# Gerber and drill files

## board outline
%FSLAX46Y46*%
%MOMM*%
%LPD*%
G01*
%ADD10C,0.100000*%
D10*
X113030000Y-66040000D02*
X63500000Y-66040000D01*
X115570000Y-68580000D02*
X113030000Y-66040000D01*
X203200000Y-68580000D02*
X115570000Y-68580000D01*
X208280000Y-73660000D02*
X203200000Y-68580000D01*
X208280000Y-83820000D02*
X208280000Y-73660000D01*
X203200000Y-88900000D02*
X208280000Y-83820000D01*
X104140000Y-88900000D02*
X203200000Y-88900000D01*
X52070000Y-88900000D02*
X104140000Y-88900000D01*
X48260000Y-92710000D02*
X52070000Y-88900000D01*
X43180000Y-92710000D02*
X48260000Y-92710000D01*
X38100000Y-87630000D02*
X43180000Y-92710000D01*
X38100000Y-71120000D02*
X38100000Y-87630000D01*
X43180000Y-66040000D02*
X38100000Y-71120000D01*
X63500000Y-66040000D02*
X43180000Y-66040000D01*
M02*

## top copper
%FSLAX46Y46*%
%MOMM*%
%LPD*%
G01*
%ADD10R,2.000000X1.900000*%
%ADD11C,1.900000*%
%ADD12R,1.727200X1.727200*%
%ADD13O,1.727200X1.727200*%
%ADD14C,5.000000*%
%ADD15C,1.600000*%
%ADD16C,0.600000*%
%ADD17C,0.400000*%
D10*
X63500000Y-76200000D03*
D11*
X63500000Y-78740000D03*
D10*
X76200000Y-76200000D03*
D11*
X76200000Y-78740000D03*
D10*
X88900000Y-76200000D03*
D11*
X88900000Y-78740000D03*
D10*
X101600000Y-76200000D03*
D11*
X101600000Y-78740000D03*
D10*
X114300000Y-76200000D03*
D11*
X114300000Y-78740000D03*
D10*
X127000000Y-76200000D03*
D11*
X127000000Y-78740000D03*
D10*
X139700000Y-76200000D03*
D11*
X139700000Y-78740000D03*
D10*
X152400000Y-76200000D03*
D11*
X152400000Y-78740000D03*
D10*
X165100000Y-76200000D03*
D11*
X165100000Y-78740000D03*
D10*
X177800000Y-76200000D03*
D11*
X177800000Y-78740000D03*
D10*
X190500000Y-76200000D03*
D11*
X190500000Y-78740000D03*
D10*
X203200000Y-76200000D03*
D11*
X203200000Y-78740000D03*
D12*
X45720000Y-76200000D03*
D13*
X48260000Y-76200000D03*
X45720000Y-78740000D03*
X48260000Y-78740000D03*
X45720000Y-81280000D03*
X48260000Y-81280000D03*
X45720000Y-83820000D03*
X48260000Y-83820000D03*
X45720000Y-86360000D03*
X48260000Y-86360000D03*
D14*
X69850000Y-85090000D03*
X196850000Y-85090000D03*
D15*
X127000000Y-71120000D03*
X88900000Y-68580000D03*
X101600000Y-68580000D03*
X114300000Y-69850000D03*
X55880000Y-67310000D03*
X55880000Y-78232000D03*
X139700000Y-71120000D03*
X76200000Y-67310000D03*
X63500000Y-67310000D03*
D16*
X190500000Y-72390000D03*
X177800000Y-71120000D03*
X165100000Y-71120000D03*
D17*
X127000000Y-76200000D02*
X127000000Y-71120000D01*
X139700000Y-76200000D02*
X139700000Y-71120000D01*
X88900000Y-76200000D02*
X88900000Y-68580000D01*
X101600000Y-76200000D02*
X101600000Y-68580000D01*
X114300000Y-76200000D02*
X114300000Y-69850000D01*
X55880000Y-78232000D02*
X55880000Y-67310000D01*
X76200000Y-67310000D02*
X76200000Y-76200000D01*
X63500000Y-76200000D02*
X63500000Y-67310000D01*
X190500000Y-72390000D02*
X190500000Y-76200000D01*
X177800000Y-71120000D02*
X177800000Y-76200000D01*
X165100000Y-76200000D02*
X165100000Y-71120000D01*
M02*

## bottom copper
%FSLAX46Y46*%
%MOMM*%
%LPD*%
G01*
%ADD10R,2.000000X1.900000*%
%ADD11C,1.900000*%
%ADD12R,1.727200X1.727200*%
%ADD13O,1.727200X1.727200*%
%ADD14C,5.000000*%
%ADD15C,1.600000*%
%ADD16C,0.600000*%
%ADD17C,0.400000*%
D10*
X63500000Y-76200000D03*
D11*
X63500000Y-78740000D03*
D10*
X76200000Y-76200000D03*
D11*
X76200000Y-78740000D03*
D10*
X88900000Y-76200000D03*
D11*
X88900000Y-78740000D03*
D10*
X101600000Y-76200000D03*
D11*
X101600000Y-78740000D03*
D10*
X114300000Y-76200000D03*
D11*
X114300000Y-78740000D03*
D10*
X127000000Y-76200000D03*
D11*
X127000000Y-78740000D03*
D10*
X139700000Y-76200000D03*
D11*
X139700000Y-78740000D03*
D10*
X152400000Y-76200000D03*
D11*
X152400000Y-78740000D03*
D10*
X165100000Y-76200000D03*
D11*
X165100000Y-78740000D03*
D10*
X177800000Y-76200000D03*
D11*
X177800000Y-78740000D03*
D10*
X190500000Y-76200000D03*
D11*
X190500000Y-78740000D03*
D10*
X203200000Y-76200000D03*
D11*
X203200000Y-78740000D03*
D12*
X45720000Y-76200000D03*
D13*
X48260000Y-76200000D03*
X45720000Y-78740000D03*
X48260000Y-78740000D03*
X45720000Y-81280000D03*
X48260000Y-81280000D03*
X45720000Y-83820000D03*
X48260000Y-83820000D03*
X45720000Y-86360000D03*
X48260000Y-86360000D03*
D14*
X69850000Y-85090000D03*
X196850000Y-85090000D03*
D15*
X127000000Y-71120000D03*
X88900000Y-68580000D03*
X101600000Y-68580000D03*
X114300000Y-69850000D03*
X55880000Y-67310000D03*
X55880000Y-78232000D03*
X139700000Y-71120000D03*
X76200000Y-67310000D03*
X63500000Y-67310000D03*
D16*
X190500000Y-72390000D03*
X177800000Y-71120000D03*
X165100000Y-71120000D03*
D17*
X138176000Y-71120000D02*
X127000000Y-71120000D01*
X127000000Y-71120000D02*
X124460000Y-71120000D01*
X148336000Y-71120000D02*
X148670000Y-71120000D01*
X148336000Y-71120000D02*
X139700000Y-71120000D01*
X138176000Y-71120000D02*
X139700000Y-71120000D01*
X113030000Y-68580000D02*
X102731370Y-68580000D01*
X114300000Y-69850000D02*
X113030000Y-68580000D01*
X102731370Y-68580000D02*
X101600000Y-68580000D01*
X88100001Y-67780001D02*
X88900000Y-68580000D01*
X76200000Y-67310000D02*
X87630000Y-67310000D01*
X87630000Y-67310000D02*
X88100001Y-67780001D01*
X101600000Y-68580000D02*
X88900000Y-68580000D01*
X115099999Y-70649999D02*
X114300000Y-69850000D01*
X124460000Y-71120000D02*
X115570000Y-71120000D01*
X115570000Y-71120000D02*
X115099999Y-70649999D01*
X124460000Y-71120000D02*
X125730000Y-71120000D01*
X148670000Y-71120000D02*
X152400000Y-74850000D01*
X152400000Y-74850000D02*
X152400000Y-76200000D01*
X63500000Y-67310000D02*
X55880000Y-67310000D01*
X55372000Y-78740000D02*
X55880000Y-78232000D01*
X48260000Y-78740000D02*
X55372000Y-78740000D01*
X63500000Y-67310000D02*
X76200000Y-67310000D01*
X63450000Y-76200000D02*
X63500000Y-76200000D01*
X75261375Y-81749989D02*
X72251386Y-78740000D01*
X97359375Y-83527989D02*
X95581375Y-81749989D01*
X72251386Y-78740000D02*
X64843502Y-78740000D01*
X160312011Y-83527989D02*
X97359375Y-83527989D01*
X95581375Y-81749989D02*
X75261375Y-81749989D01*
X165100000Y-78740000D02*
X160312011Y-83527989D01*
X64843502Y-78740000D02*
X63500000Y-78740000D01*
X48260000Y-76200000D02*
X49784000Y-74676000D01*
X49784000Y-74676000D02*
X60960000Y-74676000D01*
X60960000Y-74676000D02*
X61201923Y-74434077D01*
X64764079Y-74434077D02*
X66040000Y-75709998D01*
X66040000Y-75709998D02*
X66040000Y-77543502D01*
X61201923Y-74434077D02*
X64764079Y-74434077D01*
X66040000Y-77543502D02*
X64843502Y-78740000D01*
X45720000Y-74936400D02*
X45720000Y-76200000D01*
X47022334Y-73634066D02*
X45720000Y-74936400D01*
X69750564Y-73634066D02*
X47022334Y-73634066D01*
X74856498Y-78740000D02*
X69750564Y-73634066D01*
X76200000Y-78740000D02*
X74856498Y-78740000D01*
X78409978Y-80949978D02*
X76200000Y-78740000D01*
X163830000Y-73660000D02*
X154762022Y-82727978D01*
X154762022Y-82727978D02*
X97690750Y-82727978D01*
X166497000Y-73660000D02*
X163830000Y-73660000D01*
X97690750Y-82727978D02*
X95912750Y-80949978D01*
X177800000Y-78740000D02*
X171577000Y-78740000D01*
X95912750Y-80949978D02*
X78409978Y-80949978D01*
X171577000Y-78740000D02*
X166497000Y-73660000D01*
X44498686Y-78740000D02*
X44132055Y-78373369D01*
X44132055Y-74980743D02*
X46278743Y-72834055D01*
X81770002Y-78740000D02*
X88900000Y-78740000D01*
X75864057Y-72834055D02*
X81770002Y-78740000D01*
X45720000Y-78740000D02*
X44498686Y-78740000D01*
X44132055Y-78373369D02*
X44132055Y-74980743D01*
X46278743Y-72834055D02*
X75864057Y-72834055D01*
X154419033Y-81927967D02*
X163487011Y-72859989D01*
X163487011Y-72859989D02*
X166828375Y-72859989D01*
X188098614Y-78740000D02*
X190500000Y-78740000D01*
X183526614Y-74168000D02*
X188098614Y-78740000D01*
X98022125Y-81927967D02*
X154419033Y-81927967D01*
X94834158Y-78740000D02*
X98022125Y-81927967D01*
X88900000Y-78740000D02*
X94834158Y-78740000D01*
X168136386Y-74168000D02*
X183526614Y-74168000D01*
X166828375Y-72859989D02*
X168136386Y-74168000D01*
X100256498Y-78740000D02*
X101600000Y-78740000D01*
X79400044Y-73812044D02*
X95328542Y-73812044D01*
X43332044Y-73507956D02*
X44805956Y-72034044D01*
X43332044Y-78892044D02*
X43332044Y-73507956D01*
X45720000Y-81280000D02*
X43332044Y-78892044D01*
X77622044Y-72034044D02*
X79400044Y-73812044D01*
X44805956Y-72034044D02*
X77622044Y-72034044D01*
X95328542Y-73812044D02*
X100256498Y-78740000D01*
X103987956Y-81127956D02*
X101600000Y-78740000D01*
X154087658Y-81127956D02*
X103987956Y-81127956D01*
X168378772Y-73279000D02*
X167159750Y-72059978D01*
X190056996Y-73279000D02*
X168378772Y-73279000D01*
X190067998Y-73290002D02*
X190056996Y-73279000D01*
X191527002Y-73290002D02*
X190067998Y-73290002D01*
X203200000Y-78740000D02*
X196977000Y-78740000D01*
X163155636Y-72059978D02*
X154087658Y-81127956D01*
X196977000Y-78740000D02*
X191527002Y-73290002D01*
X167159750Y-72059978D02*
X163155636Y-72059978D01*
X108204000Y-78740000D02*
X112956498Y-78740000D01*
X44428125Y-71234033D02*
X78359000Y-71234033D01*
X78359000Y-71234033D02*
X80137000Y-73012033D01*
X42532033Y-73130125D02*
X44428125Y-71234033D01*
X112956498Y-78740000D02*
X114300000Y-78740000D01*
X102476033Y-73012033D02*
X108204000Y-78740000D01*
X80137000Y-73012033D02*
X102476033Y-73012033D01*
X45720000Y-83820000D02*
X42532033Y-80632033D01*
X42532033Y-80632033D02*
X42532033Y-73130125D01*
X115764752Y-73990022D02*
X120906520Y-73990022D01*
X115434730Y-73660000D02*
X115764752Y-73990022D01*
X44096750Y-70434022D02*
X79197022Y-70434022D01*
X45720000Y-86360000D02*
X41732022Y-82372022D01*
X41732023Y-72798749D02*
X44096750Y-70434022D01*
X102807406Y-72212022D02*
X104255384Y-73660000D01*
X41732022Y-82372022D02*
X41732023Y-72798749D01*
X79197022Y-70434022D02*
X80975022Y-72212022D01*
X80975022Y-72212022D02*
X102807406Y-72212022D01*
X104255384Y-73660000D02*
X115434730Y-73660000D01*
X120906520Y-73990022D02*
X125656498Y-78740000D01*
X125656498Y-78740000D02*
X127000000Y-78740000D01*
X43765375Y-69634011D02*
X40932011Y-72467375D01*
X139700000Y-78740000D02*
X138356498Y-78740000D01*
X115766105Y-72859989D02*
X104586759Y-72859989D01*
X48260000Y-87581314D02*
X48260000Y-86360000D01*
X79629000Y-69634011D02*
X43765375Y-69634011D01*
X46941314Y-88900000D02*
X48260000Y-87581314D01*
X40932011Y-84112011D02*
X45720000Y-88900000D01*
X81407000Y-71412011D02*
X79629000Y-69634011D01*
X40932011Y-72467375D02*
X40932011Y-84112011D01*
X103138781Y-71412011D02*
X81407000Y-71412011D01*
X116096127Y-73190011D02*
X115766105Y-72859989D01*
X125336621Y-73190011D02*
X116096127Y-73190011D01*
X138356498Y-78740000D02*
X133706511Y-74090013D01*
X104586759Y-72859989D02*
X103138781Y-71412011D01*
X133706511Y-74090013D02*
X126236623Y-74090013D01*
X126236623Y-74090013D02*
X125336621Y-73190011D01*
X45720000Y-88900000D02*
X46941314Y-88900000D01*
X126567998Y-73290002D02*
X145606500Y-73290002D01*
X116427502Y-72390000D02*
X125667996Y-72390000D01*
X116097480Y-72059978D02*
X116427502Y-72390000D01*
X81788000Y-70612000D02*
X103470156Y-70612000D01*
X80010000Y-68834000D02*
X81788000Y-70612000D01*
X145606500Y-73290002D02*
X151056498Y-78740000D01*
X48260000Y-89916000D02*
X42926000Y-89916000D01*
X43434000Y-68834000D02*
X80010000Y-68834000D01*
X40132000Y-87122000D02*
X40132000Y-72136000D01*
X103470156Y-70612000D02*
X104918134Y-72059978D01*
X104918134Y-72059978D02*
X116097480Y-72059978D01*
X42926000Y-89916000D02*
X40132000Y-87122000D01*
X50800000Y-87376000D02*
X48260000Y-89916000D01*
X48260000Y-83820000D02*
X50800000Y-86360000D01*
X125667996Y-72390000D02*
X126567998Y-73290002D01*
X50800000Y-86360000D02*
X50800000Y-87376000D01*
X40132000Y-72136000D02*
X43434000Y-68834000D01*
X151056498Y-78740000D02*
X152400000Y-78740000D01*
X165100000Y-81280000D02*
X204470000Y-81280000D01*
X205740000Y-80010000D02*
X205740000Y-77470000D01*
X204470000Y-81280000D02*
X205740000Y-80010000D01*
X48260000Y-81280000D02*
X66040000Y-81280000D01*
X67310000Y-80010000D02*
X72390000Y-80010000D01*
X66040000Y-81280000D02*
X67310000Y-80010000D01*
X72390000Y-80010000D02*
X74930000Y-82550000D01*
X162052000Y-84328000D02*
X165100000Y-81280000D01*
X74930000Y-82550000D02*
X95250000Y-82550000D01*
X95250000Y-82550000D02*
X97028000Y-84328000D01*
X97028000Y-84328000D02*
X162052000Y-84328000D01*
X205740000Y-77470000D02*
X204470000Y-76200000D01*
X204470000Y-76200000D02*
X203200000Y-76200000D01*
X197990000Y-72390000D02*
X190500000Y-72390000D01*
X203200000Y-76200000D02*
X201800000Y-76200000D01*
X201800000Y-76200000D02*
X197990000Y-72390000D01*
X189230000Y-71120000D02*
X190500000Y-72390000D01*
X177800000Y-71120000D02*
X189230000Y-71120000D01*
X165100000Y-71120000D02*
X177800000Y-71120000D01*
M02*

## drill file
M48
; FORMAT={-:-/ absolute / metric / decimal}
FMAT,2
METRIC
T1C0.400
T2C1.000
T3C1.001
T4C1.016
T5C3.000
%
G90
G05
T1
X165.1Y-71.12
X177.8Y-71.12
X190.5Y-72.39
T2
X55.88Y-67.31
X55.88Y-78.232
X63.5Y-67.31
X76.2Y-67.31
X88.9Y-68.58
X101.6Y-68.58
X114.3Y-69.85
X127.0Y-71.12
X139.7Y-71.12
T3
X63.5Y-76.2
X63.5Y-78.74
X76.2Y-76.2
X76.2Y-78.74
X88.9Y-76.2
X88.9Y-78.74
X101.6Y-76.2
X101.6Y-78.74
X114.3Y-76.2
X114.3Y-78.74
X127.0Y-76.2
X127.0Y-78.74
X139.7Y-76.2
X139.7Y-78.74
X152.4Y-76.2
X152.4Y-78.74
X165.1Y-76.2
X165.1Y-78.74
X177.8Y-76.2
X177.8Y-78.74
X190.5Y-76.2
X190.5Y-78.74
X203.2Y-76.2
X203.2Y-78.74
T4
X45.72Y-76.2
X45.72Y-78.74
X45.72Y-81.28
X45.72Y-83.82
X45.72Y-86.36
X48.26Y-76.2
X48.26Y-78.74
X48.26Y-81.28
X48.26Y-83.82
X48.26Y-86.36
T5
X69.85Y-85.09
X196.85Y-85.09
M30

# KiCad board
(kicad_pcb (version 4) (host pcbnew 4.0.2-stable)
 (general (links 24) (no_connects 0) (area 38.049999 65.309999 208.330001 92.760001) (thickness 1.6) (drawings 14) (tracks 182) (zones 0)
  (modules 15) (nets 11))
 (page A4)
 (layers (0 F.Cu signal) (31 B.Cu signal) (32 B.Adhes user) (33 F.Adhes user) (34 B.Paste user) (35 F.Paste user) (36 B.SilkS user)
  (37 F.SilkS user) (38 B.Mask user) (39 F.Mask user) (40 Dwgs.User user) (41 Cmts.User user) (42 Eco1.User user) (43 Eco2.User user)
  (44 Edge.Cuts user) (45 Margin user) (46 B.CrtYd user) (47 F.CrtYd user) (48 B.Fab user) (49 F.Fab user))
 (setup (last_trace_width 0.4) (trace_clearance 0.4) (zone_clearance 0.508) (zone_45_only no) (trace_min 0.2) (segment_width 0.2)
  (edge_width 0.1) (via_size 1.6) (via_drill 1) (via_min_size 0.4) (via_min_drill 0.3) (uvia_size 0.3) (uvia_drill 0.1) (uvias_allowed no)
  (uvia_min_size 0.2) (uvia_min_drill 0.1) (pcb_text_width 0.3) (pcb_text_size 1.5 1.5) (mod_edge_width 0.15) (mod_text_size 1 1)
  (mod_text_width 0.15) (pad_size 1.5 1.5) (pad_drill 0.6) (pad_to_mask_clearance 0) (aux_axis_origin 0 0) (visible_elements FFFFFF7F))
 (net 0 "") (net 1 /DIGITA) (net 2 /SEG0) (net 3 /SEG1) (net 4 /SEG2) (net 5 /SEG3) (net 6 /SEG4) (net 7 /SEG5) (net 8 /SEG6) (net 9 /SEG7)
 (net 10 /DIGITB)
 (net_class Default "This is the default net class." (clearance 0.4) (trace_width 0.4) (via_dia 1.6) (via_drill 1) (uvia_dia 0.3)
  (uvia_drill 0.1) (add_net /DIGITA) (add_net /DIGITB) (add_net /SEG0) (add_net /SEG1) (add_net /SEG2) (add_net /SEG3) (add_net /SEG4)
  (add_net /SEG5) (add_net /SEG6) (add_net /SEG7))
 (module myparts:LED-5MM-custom (layer F.Cu) (at 63.5 76.2 270)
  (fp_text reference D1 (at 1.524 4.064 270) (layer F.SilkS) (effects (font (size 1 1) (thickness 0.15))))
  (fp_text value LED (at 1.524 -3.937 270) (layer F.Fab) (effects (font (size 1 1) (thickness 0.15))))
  (pad 1 thru_hole rect (at 0 0) (size 2 1.9) (drill 1.00076) (layers *.Cu *.Mask F.SilkS) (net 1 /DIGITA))
  (pad 2 thru_hole circle (at 2.54 0 270) (size 1.9 1.9) (drill 1.00076) (layers *.Cu *.Mask F.SilkS) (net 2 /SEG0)))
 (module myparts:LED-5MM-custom (layer F.Cu) (at 76.2 76.2 270)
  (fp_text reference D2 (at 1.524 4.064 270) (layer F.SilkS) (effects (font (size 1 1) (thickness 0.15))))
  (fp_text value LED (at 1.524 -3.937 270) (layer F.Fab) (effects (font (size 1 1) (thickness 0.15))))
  (pad 1 thru_hole rect (at 0 0) (size 2 1.9) (drill 1.00076) (layers *.Cu *.Mask F.SilkS) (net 1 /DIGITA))
  (pad 2 thru_hole circle (at 2.54 0 270) (size 1.9 1.9) (drill 1.00076) (layers *.Cu *.Mask F.SilkS) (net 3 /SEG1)))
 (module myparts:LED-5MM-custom (layer F.Cu) (at 88.9 76.2 270)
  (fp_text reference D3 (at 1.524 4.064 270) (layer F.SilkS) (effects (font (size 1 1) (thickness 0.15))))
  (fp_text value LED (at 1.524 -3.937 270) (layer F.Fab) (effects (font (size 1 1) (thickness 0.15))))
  (pad 1 thru_hole rect (at 0 0) (size 2 1.9) (drill 1.00076) (layers *.Cu *.Mask F.SilkS) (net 1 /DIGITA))
  (pad 2 thru_hole circle (at 2.54 0 270) (size 1.9 1.9) (drill 1.00076) (layers *.Cu *.Mask F.SilkS) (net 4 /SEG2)))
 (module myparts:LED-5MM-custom (layer F.Cu) (at 101.6 76.2 270)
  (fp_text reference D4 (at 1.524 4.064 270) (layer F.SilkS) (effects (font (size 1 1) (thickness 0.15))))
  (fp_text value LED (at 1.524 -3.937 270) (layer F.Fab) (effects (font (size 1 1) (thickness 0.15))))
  (pad 1 thru_hole rect (at 0 0) (size 2 1.9) (drill 1.00076) (layers *.Cu *.Mask F.SilkS) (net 1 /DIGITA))
  (pad 2 thru_hole circle (at 2.54 0 270) (size 1.9 1.9) (drill 1.00076) (layers *.Cu *.Mask F.SilkS) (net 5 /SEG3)))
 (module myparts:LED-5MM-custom (layer F.Cu) (at 114.3 76.2 270)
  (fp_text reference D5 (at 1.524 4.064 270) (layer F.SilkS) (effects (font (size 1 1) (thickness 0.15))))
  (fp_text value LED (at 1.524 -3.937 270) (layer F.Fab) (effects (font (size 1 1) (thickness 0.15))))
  (pad 1 thru_hole rect (at 0 0) (size 2 1.9) (drill 1.00076) (layers *.Cu *.Mask F.SilkS) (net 1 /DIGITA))
  (pad 2 thru_hole circle (at 2.54 0 270) (size 1.9 1.9) (drill 1.00076) (layers *.Cu *.Mask F.SilkS) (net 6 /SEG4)))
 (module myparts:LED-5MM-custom (layer F.Cu) (at 127 76.2 270)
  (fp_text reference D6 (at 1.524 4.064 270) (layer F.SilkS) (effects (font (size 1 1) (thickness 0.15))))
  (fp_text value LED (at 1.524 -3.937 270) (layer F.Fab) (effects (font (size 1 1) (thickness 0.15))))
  (pad 1 thru_hole rect (at 0 0) (size 2 1.9) (drill 1.00076) (layers *.Cu *.Mask F.SilkS) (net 1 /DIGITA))
  (pad 2 thru_hole circle (at 2.54 0 270) (size 1.9 1.9) (drill 1.00076) (layers *.Cu *.Mask F.SilkS) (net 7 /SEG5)))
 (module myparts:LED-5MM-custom (layer F.Cu) (at 139.7 76.2 270)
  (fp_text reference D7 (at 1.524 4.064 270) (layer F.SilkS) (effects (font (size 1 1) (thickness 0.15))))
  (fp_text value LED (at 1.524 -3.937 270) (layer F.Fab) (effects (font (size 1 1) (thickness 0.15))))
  (pad 1 thru_hole rect (at 0 0) (size 2 1.9) (drill 1.00076) (layers *.Cu *.Mask F.SilkS) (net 1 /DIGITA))
  (pad 2 thru_hole circle (at 2.54 0 270) (size 1.9 1.9) (drill 1.00076) (layers *.Cu *.Mask F.SilkS) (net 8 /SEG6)))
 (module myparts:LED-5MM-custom (layer F.Cu) (at 152.4 76.2 270)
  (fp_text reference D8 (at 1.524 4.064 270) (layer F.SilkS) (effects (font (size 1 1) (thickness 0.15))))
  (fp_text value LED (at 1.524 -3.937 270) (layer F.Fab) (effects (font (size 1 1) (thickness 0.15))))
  (pad 1 thru_hole rect (at 0 0) (size 2 1.9) (drill 1.00076) (layers *.Cu *.Mask F.SilkS) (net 1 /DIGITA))
  (pad 2 thru_hole circle (at 2.54 0 270) (size 1.9 1.9) (drill 1.00076) (layers *.Cu *.Mask F.SilkS) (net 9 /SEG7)))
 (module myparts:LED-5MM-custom (layer F.Cu) (at 165.1 76.2 270)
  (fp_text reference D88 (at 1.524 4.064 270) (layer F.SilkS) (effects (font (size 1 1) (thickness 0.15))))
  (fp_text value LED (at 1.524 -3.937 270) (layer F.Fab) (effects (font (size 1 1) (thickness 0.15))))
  (pad 1 thru_hole rect (at 0 0) (size 2 1.9) (drill 1.00076) (layers *.Cu *.Mask F.SilkS) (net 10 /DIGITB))
  (pad 2 thru_hole circle (at 2.54 0 270) (size 1.9 1.9) (drill 1.00076) (layers *.Cu *.Mask F.SilkS) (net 2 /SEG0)))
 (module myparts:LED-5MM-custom (layer F.Cu) (at 177.8 76.2 270)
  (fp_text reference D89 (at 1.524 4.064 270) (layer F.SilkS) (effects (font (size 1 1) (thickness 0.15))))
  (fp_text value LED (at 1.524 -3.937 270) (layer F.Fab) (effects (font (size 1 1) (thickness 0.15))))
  (pad 1 thru_hole rect (at 0 0) (size 2 1.9) (drill 1.00076) (layers *.Cu *.Mask F.SilkS) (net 10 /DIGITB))
  (pad 2 thru_hole circle (at 2.54 0 270) (size 1.9 1.9) (drill 1.00076) (layers *.Cu *.Mask F.SilkS) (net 3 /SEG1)))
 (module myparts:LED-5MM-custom (layer F.Cu) (at 190.5 76.2 270)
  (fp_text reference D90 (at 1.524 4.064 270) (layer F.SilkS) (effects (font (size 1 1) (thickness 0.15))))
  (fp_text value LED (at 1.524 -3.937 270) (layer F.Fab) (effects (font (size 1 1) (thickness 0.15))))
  (pad 1 thru_hole rect (at 0 0) (size 2 1.9) (drill 1.00076) (layers *.Cu *.Mask F.SilkS) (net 10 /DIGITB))
  (pad 2 thru_hole circle (at 2.54 0 270) (size 1.9 1.9) (drill 1.00076) (layers *.Cu *.Mask F.SilkS) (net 4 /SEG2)))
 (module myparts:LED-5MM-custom (layer F.Cu) (at 203.2 76.2 270)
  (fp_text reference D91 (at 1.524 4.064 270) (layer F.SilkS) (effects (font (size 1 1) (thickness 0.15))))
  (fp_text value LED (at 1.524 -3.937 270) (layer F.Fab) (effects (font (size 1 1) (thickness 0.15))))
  (pad 1 thru_hole rect (at 0 0) (size 2 1.9) (drill 1.00076) (layers *.Cu *.Mask F.SilkS) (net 10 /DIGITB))
  (pad 2 thru_hole circle (at 2.54 0 270) (size 1.9 1.9) (drill 1.00076) (layers *.Cu *.Mask F.SilkS) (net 5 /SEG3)))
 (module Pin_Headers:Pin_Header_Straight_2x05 (layer F.Cu) (at 45.72 76.2)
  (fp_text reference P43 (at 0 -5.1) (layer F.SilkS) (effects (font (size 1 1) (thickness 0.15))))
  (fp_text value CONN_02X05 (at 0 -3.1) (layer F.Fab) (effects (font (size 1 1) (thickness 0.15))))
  (pad 1 thru_hole rect (at 0 0) (size 1.7272 1.7272) (drill 1.016) (layers *.Cu *.Mask F.SilkS) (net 3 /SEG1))
  (pad 2 thru_hole oval (at 2.54 0) (size 1.7272 1.7272) (drill 1.016) (layers *.Cu *.Mask F.SilkS) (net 2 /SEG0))
  (pad 3 thru_hole oval (at 0 2.54) (size 1.7272 1.7272) (drill 1.016) (layers *.Cu *.Mask F.SilkS) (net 4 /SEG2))
  (pad 4 thru_hole oval (at 2.54 2.54) (size 1.7272 1.7272) (drill 1.016) (layers *.Cu *.Mask F.SilkS) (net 1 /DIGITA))
  (pad 5 thru_hole oval (at 0 5.08) (size 1.7272 1.7272) (drill 1.016) (layers *.Cu *.Mask F.SilkS) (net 5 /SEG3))
  (pad 6 thru_hole oval (at 2.54 5.08) (size 1.7272 1.7272) (drill 1.016) (layers *.Cu *.Mask F.SilkS) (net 10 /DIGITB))
  (pad 7 thru_hole oval (at 0 7.62) (size 1.7272 1.7272) (drill 1.016) (layers *.Cu *.Mask F.SilkS) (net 6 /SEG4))
  (pad 8 thru_hole oval (at 2.54 7.62) (size 1.7272 1.7272) (drill 1.016) (layers *.Cu *.Mask F.SilkS) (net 9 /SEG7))
  (pad 9 thru_hole oval (at 0 10.16) (size 1.7272 1.7272) (drill 1.016) (layers *.Cu *.Mask F.SilkS) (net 7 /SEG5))
  (pad 10 thru_hole oval (at 2.54 10.16) (size 1.7272 1.7272) (drill 1.016) (layers *.Cu *.Mask F.SilkS) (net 8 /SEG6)))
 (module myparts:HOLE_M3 (layer F.Cu) (at 69.85 85.09)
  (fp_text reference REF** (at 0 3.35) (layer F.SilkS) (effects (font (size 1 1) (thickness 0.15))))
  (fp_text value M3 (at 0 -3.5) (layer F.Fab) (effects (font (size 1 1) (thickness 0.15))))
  (pad 1 thru_hole circle (at 0 0) (size 5 5) (drill 3) (layers *.Cu *.Mask F.SilkS)))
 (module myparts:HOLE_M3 (layer F.Cu) (at 196.85 85.09)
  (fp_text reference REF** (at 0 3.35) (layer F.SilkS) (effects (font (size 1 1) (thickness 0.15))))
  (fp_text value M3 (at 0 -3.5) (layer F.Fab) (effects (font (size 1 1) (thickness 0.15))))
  (pad 1 thru_hole circle (at 0 0) (size 5 5) (drill 3) (layers *.Cu *.Mask F.SilkS)))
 (gr_line (start 113.03 66.04) (end 63.5 66.04) (layer Edge.Cuts) (width 0.1))
 (gr_line (start 115.57 68.58) (end 113.03 66.04) (layer Edge.Cuts) (width 0.1))
 (gr_line (start 203.2 68.58) (end 115.57 68.58) (layer Edge.Cuts) (width 0.1))
 (gr_line (start 208.28 73.66) (end 203.2 68.58) (layer Edge.Cuts) (width 0.1))
 (gr_line (start 208.28 83.82) (end 208.28 73.66) (layer Edge.Cuts) (width 0.1))
 (gr_line (start 203.2 88.9) (end 208.28 83.82) (layer Edge.Cuts) (width 0.1))
 (gr_line (start 104.14 88.9) (end 203.2 88.9) (layer Edge.Cuts) (width 0.1))
 (gr_line (start 52.07 88.9) (end 104.14 88.9) (layer Edge.Cuts) (width 0.1))
 (gr_line (start 48.26 92.71) (end 52.07 88.9) (layer Edge.Cuts) (width 0.1))
 (gr_line (start 43.18 92.71) (end 48.26 92.71) (layer Edge.Cuts) (width 0.1))
 (gr_line (start 38.1 87.63) (end 43.18 92.71) (layer Edge.Cuts) (width 0.1))
 (gr_line (start 38.1 71.12) (end 38.1 87.63) (layer Edge.Cuts) (width 0.1))
 (gr_line (start 43.18 66.04) (end 38.1 71.12) (layer Edge.Cuts) (width 0.1))
 (gr_line (start 63.5 66.04) (end 43.18 66.04) (layer Edge.Cuts) (width 0.1))
 (segment (start 138.176 71.12) (end 127 71.12) (width 0.4) (layer B.Cu) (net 1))
 (segment (start 127 71.12) (end 124.46 71.12) (width 0.4) (layer B.Cu) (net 1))
 (segment (start 127 76.2) (end 127 71.12) (width 0.4) (layer F.Cu) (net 1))
 (via (at 127 71.12) (size 1.6) (drill 1) (layers F.Cu B.Cu) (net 1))
 (segment (start 148.336 71.12) (end 148.67 71.12) (width 0.4) (layer B.Cu) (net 1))
 (segment (start 148.336 71.12) (end 139.7 71.12) (width 0.4) (layer B.Cu) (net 1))
 (segment (start 138.176 71.12) (end 139.7 71.12) (width 0.4) (layer B.Cu) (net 1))
 (segment (start 139.7 76.2) (end 139.7 71.12) (width 0.4) (layer F.Cu) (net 1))
 (segment (start 113.03 68.58) (end 102.73137 68.58) (width 0.4) (layer B.Cu) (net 1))
 (segment (start 114.3 69.85) (end 113.03 68.58) (width 0.4) (layer B.Cu) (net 1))
 (segment (start 102.73137 68.58) (end 101.6 68.58) (width 0.4) (layer B.Cu) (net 1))
 (segment (start 88.100001 67.780001) (end 88.9 68.58) (width 0.4) (layer B.Cu) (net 1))
 (via (at 88.9 68.58) (size 1.6) (drill 1) (layers F.Cu B.Cu) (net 1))
 (segment (start 76.2 67.31) (end 87.63 67.31) (width 0.4) (layer B.Cu) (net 1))
 (segment (start 87.63 67.31) (end 88.100001 67.780001) (width 0.4) (layer B.Cu) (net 1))
 (segment (start 88.9 76.2) (end 88.9 68.58) (width 0.4) (layer F.Cu) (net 1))
 (segment (start 101.6 68.58) (end 88.9 68.58) (width 0.4) (layer B.Cu) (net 1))
 (via (at 101.6 68.58) (size 1.6) (drill 1) (layers F.Cu B.Cu) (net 1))
 (segment (start 101.6 76.2) (end 101.6 68.58) (width 0.4) (layer F.Cu) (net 1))
 (segment (start 115.099999 70.649999) (end 114.3 69.85) (width 0.4) (layer B.Cu) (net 1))
 (segment (start 124.46 71.12) (end 115.57 71.12) (width 0.4) (layer B.Cu) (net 1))
 (segment (start 114.3 76.2) (end 114.3 69.85) (width 0.4) (layer F.Cu) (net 1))
 (segment (start 115.57 71.12) (end 115.099999 70.649999) (width 0.4) (layer B.Cu) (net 1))
 (via (at 114.3 69.85) (size 1.6) (drill 1) (layers F.Cu B.Cu) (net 1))
 (segment (start 124.46 71.12) (end 125.73 71.12) (width 0.4) (layer B.Cu) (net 1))
 (segment (start 148.67 71.12) (end 152.4 74.85) (width 0.4) (layer B.Cu) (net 1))
 (segment (start 152.4 74.85) (end 152.4 76.2) (width 0.4) (layer B.Cu) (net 1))
 (segment (start 55.88 78.232) (end 55.88 67.31) (width 0.4) (layer F.Cu) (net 1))
 (segment (start 63.5 67.31) (end 55.88 67.31) (width 0.4) (layer B.Cu) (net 1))
 (via (at 55.88 67.31) (size 1.6) (drill 1) (layers F.Cu B.Cu) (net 1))
 (segment (start 55.372 78.74) (end 55.88 78.232) (width 0.4) (layer B.Cu) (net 1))
 (segment (start 48.26 78.74) (end 55.372 78.74) (width 0.4) (layer B.Cu) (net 1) (status 10))
 (via (at 55.88 78.232) (size 1.6) (drill 1) (layers F.Cu B.Cu) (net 1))
 (via (at 139.7 71.12) (size 1.6) (drill 1) (layers F.Cu B.Cu) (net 1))
 (segment (start 76.2 67.31) (end 76.2 76.2) (width 0.4) (layer F.Cu) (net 1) (status 20))
 (segment (start 63.5 67.31) (end 76.2 67.31) (width 0.4) (layer B.Cu) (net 1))
 (via (at 76.2 67.31) (size 1.6) (drill 1) (layers F.Cu B.Cu) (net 1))
 (segment (start 63.5 76.2) (end 63.5 67.31) (width 0.4) (layer F.Cu) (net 1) (status 10))
 (via (at 63.5 67.31) (size 1.6) (drill 1) (layers F.Cu B.Cu) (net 1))
 (segment (start 63.45 76.2) (end 63.5 76.2) (width 0.4) (layer B.Cu) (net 1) (status 30))
 (segment (start 75.261375 81.749989) (end 72.251386 78.74) (width 0.4) (layer B.Cu) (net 2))
 (segment (start 97.359375 83.527989) (end 95.581375 81.749989) (width 0.4) (layer B.Cu) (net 2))
 (segment (start 72.251386 78.74) (end 64.843502 78.74) (width 0.4) (layer B.Cu) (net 2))
 (segment (start 160.312011 83.527989) (end 97.359375 83.527989) (width 0.4) (layer B.Cu) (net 2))
 (segment (start 95.581375 81.749989) (end 75.261375 81.749989) (width 0.4) (layer B.Cu) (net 2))
 (segment (start 165.1 78.74) (end 160.312011 83.527989) (width 0.4) (layer B.Cu) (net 2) (status 10))
 (segment (start 64.843502 78.74) (end 63.5 78.74) (width 0.4) (layer B.Cu) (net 2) (status 20))
 (segment (start 48.26 76.2) (end 49.784 74.676) (width 0.4) (layer B.Cu) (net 2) (status 10))
 (segment (start 49.784 74.676) (end 60.96 74.676) (width 0.4) (layer B.Cu) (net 2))
 (segment (start 60.96 74.676) (end 61.201923 74.434077) (width 0.4) (layer B.Cu) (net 2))
 (segment (start 64.764079 74.434077) (end 66.04 75.709998) (width 0.4) (layer B.Cu) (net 2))
 (segment (start 66.04 75.709998) (end 66.04 77.543502) (width 0.4) (layer B.Cu) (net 2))
 (segment (start 61.201923 74.434077) (end 64.764079 74.434077) (width 0.4) (layer B.Cu) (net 2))
 (segment (start 66.04 77.543502) (end 64.843502 78.74) (width 0.4) (layer B.Cu) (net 2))
 (segment (start 45.72 74.9364) (end 45.72 76.2) (width 0.4) (layer B.Cu) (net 3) (status 20))
 (segment (start 47.022334 73.634066) (end 45.72 74.9364) (width 0.4) (layer B.Cu) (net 3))
 (segment (start 69.750564 73.634066) (end 47.022334 73.634066) (width 0.4) (layer B.Cu) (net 3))
 (segment (start 74.856498 78.74) (end 69.750564 73.634066) (width 0.4) (layer B.Cu) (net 3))
 (segment (start 76.2 78.74) (end 74.856498 78.74) (width 0.4) (layer B.Cu) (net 3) (status 10))
 (segment (start 78.409978 80.949978) (end 76.2 78.74) (width 0.4) (layer B.Cu) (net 3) (status 20))
 (segment (start 163.83 73.66) (end 154.762022 82.727978) (width 0.4) (layer B.Cu) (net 3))
 (segment (start 154.762022 82.727978) (end 97.69075 82.727978) (width 0.4) (layer B.Cu) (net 3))
 (segment (start 166.497 73.66) (end 163.83 73.66) (width 0.4) (layer B.Cu) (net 3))
 (segment (start 97.69075 82.727978) (end 95.91275 80.949978) (width 0.4) (layer B.Cu) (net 3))
 (segment (start 177.8 78.74) (end 171.577 78.74) (width 0.4) (layer B.Cu) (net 3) (status 10))
 (segment (start 95.91275 80.949978) (end 78.409978 80.949978) (width 0.4) (layer B.Cu) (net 3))
 (segment (start 171.577 78.74) (end 166.497 73.66) (width 0.4) (layer B.Cu) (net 3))
 (segment (start 44.498686 78.74) (end 44.132055 78.373369) (width 0.4) (layer B.Cu) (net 4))
 (segment (start 44.132055 74.980743) (end 46.278743 72.834055) (width 0.4) (layer B.Cu) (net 4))
 (segment (start 81.770002 78.74) (end 88.9 78.74) (width 0.4) (layer B.Cu) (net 4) (status 20))
 (segment (start 75.864057 72.834055) (end 81.770002 78.74) (width 0.4) (layer B.Cu) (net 4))
 (segment (start 45.72 78.74) (end 44.498686 78.74) (width 0.4) (layer B.Cu) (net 4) (status 10))
 (segment (start 44.132055 78.373369) (end 44.132055 74.980743) (width 0.4) (layer B.Cu) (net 4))
 (segment (start 46.278743 72.834055) (end 75.864057 72.834055) (width 0.4) (layer B.Cu) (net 4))
 (segment (start 154.419033 81.927967) (end 163.487011 72.859989) (width 0.4) (layer B.Cu) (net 4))
 (segment (start 163.487011 72.859989) (end 166.828375 72.859989) (width 0.4) (layer B.Cu) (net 4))
 (segment (start 188.098614 78.74) (end 190.5 78.74) (width 0.4) (layer B.Cu) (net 4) (status 20))
 (segment (start 183.526614 74.168) (end 188.098614 78.74) (width 0.4) (layer B.Cu) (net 4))
 (segment (start 98.022125 81.927967) (end 154.419033 81.927967) (width 0.4) (layer B.Cu) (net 4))
 (segment (start 94.834158 78.74) (end 98.022125 81.927967) (width 0.4) (layer B.Cu) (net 4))
 (segment (start 88.9 78.74) (end 94.834158 78.74) (width 0.4) (layer B.Cu) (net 4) (status 10))
 (segment (start 168.136386 74.168) (end 183.526614 74.168) (width 0.4) (layer B.Cu) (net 4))
 (segment (start 166.828375 72.859989) (end 168.136386 74.168) (width 0.4) (layer B.Cu) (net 4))
 (segment (start 100.256498 78.74) (end 101.6 78.74) (width 0.4) (layer B.Cu) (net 5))
 (segment (start 79.400044 73.812044) (end 95.328542 73.812044) (width 0.4) (layer B.Cu) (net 5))
 (segment (start 43.332044 73.507956) (end 44.805956 72.034044) (width 0.4) (layer B.Cu) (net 5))
 (segment (start 43.332044 78.892044) (end 43.332044 73.507956) (width 0.4) (layer B.Cu) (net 5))
 (segment (start 45.72 81.28) (end 43.332044 78.892044) (width 0.4) (layer B.Cu) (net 5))
 (segment (start 77.622044 72.034044) (end 79.400044 73.812044) (width 0.4) (layer B.Cu) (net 5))
 (segment (start 44.805956 72.034044) (end 77.622044 72.034044) (width 0.4) (layer B.Cu) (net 5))
 (segment (start 95.328542 73.812044) (end 100.256498 78.74) (width 0.4) (layer B.Cu) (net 5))
 (segment (start 103.987956 81.127956) (end 101.6 78.74) (width 0.4) (layer B.Cu) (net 5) (status 20))
 (segment (start 154.087658 81.127956) (end 103.987956 81.127956) (width 0.4) (layer B.Cu) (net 5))
 (segment (start 168.378772 73.279) (end 167.15975 72.059978) (width 0.4) (layer B.Cu) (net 5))
 (segment (start 190.056996 73.279) (end 168.378772 73.279) (width 0.4) (layer B.Cu) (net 5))
 (segment (start 190.067998 73.290002) (end 190.056996 73.279) (width 0.4) (layer B.Cu) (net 5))
 (segment (start 191.527002 73.290002) (end 190.067998 73.290002) (width 0.4) (layer B.Cu) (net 5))
 (segment (start 203.2 78.74) (end 196.977 78.74) (width 0.4) (layer B.Cu) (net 5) (status 10))
 (segment (start 163.155636 72.059978) (end 154.087658 81.127956) (width 0.4) (layer B.Cu) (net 5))
 (segment (start 196.977 78.74) (end 191.527002 73.290002) (width 0.4) (layer B.Cu) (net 5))
 (segment (start 167.15975 72.059978) (end 163.155636 72.059978) (width 0.4) (layer B.Cu) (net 5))
 (segment (start 108.204 78.74) (end 112.956498 78.74) (width 0.4) (layer B.Cu) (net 6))
 (segment (start 44.428125 71.234033) (end 78.359 71.234033) (width 0.4) (layer B.Cu) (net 6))
 (segment (start 78.359 71.234033) (end 80.137 73.012033) (width 0.4) (layer B.Cu) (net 6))
 (segment (start 42.532033 73.130125) (end 44.428125 71.234033) (width 0.4) (layer B.Cu) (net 6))
 (segment (start 112.956498 78.74) (end 114.3 78.74) (width 0.4) (layer B.Cu) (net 6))
 (segment (start 102.476033 73.012033) (end 108.204 78.74) (width 0.4) (layer B.Cu) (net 6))
 (segment (start 80.137 73.012033) (end 102.476033 73.012033) (width 0.4) (layer B.Cu) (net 6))
 (segment (start 45.72 83.82) (end 42.532033 80.632033) (width 0.4) (layer B.Cu) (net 6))
 (segment (start 42.532033 80.632033) (end 42.532033 73.130125) (width 0.4) (layer B.Cu) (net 6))
 (segment (start 115.764752 73.990022) (end 120.90652 73.990022) (width 0.4) (layer B.Cu) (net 7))
 (segment (start 115.43473 73.66) (end 115.764752 73.990022) (width 0.4) (layer B.Cu) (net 7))
 (segment (start 44.09675 70.434022) (end 79.197022 70.434022) (width 0.4) (layer B.Cu) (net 7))
 (segment (start 45.72 86.36) (end 41.732022 82.372022) (width 0.4) (layer B.Cu) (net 7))
 (segment (start 41.732023 72.798749) (end 44.09675 70.434022) (width 0.4) (layer B.Cu) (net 7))
 (segment (start 102.807406 72.212022) (end 104.255384 73.66) (width 0.4) (layer B.Cu) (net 7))
 (segment (start 41.732022 82.372022) (end 41.732023 72.798749) (width 0.4) (layer B.Cu) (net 7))
 (segment (start 79.197022 70.434022) (end 80.975022 72.212022) (width 0.4) (layer B.Cu) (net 7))
 (segment (start 80.975022 72.212022) (end 102.807406 72.212022) (width 0.4) (layer B.Cu) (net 7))
 (segment (start 104.255384 73.66) (end 115.43473 73.66) (width 0.4) (layer B.Cu) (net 7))
 (segment (start 120.90652 73.990022) (end 125.656498 78.74) (width 0.4) (layer B.Cu) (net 7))
 (segment (start 125.656498 78.74) (end 127 78.74) (width 0.4) (layer B.Cu) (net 7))
 (segment (start 43.765375 69.634011) (end 40.932011 72.467375) (width 0.4) (layer B.Cu) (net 8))
 (segment (start 139.7 78.74) (end 138.356498 78.74) (width 0.4) (layer B.Cu) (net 8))
 (segment (start 115.766105 72.859989) (end 104.586759 72.859989) (width 0.4) (layer B.Cu) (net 8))
 (segment (start 48.26 87.581314) (end 48.26 86.36) (width 0.4) (layer B.Cu) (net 8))
 (segment (start 79.629 69.634011) (end 43.765375 69.634011) (width 0.4) (layer B.Cu) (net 8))
 (segment (start 46.941314 88.9) (end 48.26 87.581314) (width 0.4) (layer B.Cu) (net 8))
 (segment (start 40.932011 84.112011) (end 45.72 88.9) (width 0.4) (layer B.Cu) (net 8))
 (segment (start 81.407 71.412011) (end 79.629 69.634011) (width 0.4) (layer B.Cu) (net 8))
 (segment (start 40.932011 72.467375) (end 40.932011 84.112011) (width 0.4) (layer B.Cu) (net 8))
 (segment (start 103.138781 71.412011) (end 81.407 71.412011) (width 0.4) (layer B.Cu) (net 8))
 (segment (start 116.096127 73.190011) (end 115.766105 72.859989) (width 0.4) (layer B.Cu) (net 8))
 (segment (start 125.336621 73.190011) (end 116.096127 73.190011) (width 0.4) (layer B.Cu) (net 8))
 (segment (start 138.356498 78.74) (end 133.706511 74.090013) (width 0.4) (layer B.Cu) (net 8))
 (segment (start 104.586759 72.859989) (end 103.138781 71.412011) (width 0.4) (layer B.Cu) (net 8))
 (segment (start 133.706511 74.090013) (end 126.236623 74.090013) (width 0.4) (layer B.Cu) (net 8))
 (segment (start 126.236623 74.090013) (end 125.336621 73.190011) (width 0.4) (layer B.Cu) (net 8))
 (segment (start 45.72 88.9) (end 46.941314 88.9) (width 0.4) (layer B.Cu) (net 8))
 (segment (start 126.567998 73.290002) (end 145.6065 73.290002) (width 0.4) (layer B.Cu) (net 9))
 (segment (start 116.427502 72.39) (end 125.667996 72.39) (width 0.4) (layer B.Cu) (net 9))
 (segment (start 116.09748 72.059978) (end 116.427502 72.39) (width 0.4) (layer B.Cu) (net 9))
 (segment (start 81.788 70.612) (end 103.470156 70.612) (width 0.4) (layer B.Cu) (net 9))
 (segment (start 80.01 68.834) (end 81.788 70.612) (width 0.4) (layer B.Cu) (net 9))
 (segment (start 145.6065 73.290002) (end 151.056498 78.74) (width 0.4) (layer B.Cu) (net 9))
 (segment (start 48.26 89.916) (end 42.926 89.916) (width 0.4) (layer B.Cu) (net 9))
 (segment (start 43.434 68.834) (end 80.01 68.834) (width 0.4) (layer B.Cu) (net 9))
 (segment (start 40.132 87.122) (end 40.132 72.136) (width 0.4) (layer B.Cu) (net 9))
 (segment (start 103.470156 70.612) (end 104.918134 72.059978) (width 0.4) (layer B.Cu) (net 9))
 (segment (start 104.918134 72.059978) (end 116.09748 72.059978) (width 0.4) (layer B.Cu) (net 9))
 (segment (start 42.926 89.916) (end 40.132 87.122) (width 0.4) (layer B.Cu) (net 9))
 (segment (start 50.8 87.376) (end 48.26 89.916) (width 0.4) (layer B.Cu) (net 9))
 (segment (start 48.26 83.82) (end 50.8 86.36) (width 0.4) (layer B.Cu) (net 9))
 (segment (start 125.667996 72.39) (end 126.567998 73.290002) (width 0.4) (layer B.Cu) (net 9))
 (segment (start 50.8 86.36) (end 50.8 87.376) (width 0.4) (layer B.Cu) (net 9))
 (segment (start 40.132 72.136) (end 43.434 68.834) (width 0.4) (layer B.Cu) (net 9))
 (segment (start 151.056498 78.74) (end 152.4 78.74) (width 0.4) (layer B.Cu) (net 9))
 (segment (start 165.1 81.28) (end 204.47 81.28) (width 0.4) (layer B.Cu) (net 10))
 (segment (start 205.74 80.01) (end 205.74 77.47) (width 0.4) (layer B.Cu) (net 10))
 (segment (start 204.47 81.28) (end 205.74 80.01) (width 0.4) (layer B.Cu) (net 10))
 (segment (start 48.26 81.28) (end 66.04 81.28) (width 0.4) (layer B.Cu) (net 10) (status 10))
 (segment (start 67.31 80.01) (end 72.39 80.01) (width 0.4) (layer B.Cu) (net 10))
 (segment (start 66.04 81.28) (end 67.31 80.01) (width 0.4) (layer B.Cu) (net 10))
 (segment (start 72.39 80.01) (end 74.93 82.55) (width 0.4) (layer B.Cu) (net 10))
 (segment (start 162.052 84.328) (end 165.1 81.28) (width 0.4) (layer B.Cu) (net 10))
 (segment (start 74.93 82.55) (end 95.25 82.55) (width 0.4) (layer B.Cu) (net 10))
 (segment (start 95.25 82.55) (end 97.028 84.328) (width 0.4) (layer B.Cu) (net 10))
 (segment (start 97.028 84.328) (end 162.052 84.328) (width 0.4) (layer B.Cu) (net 10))
 (segment (start 205.74 77.47) (end 204.47 76.2) (width 0.4) (layer B.Cu) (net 10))
 (segment (start 204.47 76.2) (end 203.2 76.2) (width 0.4) (layer B.Cu) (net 10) (status 20))
 (segment (start 197.99 72.39) (end 190.5 72.39) (width 0.4) (layer B.Cu) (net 10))
 (segment (start 203.2 76.2) (end 201.8 76.2) (width 0.4) (layer B.Cu) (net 10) (status 10))
 (segment (start 201.8 76.2) (end 197.99 72.39) (width 0.4) (layer B.Cu) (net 10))
 (segment (start 190.5 72.39) (end 190.5 76.2) (width 0.4) (layer F.Cu) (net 10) (status 20))
 (segment (start 189.23 71.12) (end 190.5 72.39) (width 0.4) (layer B.Cu) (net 10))
 (via (at 190.5 72.39) (size 0.6) (drill 0.4) (layers F.Cu B.Cu) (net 10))
 (segment (start 177.8 71.12) (end 189.23 71.12) (width 0.4) (layer B.Cu) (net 10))
 (segment (start 177.8 71.12) (end 177.8 76.2) (width 0.4) (layer F.Cu) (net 10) (status 20))
 (segment (start 165.1 71.12) (end 177.8 71.12) (width 0.4) (layer B.Cu) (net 10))
 (via (at 177.8 71.12) (size 0.6) (drill 0.4) (layers F.Cu B.Cu) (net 10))
 (segment (start 165.1 76.2) (end 165.1 71.12) (width 0.4) (layer F.Cu) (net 10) (status 10))
 (via (at 165.1 71.12) (size 0.6) (drill 0.4) (layers F.Cu B.Cu) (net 10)))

